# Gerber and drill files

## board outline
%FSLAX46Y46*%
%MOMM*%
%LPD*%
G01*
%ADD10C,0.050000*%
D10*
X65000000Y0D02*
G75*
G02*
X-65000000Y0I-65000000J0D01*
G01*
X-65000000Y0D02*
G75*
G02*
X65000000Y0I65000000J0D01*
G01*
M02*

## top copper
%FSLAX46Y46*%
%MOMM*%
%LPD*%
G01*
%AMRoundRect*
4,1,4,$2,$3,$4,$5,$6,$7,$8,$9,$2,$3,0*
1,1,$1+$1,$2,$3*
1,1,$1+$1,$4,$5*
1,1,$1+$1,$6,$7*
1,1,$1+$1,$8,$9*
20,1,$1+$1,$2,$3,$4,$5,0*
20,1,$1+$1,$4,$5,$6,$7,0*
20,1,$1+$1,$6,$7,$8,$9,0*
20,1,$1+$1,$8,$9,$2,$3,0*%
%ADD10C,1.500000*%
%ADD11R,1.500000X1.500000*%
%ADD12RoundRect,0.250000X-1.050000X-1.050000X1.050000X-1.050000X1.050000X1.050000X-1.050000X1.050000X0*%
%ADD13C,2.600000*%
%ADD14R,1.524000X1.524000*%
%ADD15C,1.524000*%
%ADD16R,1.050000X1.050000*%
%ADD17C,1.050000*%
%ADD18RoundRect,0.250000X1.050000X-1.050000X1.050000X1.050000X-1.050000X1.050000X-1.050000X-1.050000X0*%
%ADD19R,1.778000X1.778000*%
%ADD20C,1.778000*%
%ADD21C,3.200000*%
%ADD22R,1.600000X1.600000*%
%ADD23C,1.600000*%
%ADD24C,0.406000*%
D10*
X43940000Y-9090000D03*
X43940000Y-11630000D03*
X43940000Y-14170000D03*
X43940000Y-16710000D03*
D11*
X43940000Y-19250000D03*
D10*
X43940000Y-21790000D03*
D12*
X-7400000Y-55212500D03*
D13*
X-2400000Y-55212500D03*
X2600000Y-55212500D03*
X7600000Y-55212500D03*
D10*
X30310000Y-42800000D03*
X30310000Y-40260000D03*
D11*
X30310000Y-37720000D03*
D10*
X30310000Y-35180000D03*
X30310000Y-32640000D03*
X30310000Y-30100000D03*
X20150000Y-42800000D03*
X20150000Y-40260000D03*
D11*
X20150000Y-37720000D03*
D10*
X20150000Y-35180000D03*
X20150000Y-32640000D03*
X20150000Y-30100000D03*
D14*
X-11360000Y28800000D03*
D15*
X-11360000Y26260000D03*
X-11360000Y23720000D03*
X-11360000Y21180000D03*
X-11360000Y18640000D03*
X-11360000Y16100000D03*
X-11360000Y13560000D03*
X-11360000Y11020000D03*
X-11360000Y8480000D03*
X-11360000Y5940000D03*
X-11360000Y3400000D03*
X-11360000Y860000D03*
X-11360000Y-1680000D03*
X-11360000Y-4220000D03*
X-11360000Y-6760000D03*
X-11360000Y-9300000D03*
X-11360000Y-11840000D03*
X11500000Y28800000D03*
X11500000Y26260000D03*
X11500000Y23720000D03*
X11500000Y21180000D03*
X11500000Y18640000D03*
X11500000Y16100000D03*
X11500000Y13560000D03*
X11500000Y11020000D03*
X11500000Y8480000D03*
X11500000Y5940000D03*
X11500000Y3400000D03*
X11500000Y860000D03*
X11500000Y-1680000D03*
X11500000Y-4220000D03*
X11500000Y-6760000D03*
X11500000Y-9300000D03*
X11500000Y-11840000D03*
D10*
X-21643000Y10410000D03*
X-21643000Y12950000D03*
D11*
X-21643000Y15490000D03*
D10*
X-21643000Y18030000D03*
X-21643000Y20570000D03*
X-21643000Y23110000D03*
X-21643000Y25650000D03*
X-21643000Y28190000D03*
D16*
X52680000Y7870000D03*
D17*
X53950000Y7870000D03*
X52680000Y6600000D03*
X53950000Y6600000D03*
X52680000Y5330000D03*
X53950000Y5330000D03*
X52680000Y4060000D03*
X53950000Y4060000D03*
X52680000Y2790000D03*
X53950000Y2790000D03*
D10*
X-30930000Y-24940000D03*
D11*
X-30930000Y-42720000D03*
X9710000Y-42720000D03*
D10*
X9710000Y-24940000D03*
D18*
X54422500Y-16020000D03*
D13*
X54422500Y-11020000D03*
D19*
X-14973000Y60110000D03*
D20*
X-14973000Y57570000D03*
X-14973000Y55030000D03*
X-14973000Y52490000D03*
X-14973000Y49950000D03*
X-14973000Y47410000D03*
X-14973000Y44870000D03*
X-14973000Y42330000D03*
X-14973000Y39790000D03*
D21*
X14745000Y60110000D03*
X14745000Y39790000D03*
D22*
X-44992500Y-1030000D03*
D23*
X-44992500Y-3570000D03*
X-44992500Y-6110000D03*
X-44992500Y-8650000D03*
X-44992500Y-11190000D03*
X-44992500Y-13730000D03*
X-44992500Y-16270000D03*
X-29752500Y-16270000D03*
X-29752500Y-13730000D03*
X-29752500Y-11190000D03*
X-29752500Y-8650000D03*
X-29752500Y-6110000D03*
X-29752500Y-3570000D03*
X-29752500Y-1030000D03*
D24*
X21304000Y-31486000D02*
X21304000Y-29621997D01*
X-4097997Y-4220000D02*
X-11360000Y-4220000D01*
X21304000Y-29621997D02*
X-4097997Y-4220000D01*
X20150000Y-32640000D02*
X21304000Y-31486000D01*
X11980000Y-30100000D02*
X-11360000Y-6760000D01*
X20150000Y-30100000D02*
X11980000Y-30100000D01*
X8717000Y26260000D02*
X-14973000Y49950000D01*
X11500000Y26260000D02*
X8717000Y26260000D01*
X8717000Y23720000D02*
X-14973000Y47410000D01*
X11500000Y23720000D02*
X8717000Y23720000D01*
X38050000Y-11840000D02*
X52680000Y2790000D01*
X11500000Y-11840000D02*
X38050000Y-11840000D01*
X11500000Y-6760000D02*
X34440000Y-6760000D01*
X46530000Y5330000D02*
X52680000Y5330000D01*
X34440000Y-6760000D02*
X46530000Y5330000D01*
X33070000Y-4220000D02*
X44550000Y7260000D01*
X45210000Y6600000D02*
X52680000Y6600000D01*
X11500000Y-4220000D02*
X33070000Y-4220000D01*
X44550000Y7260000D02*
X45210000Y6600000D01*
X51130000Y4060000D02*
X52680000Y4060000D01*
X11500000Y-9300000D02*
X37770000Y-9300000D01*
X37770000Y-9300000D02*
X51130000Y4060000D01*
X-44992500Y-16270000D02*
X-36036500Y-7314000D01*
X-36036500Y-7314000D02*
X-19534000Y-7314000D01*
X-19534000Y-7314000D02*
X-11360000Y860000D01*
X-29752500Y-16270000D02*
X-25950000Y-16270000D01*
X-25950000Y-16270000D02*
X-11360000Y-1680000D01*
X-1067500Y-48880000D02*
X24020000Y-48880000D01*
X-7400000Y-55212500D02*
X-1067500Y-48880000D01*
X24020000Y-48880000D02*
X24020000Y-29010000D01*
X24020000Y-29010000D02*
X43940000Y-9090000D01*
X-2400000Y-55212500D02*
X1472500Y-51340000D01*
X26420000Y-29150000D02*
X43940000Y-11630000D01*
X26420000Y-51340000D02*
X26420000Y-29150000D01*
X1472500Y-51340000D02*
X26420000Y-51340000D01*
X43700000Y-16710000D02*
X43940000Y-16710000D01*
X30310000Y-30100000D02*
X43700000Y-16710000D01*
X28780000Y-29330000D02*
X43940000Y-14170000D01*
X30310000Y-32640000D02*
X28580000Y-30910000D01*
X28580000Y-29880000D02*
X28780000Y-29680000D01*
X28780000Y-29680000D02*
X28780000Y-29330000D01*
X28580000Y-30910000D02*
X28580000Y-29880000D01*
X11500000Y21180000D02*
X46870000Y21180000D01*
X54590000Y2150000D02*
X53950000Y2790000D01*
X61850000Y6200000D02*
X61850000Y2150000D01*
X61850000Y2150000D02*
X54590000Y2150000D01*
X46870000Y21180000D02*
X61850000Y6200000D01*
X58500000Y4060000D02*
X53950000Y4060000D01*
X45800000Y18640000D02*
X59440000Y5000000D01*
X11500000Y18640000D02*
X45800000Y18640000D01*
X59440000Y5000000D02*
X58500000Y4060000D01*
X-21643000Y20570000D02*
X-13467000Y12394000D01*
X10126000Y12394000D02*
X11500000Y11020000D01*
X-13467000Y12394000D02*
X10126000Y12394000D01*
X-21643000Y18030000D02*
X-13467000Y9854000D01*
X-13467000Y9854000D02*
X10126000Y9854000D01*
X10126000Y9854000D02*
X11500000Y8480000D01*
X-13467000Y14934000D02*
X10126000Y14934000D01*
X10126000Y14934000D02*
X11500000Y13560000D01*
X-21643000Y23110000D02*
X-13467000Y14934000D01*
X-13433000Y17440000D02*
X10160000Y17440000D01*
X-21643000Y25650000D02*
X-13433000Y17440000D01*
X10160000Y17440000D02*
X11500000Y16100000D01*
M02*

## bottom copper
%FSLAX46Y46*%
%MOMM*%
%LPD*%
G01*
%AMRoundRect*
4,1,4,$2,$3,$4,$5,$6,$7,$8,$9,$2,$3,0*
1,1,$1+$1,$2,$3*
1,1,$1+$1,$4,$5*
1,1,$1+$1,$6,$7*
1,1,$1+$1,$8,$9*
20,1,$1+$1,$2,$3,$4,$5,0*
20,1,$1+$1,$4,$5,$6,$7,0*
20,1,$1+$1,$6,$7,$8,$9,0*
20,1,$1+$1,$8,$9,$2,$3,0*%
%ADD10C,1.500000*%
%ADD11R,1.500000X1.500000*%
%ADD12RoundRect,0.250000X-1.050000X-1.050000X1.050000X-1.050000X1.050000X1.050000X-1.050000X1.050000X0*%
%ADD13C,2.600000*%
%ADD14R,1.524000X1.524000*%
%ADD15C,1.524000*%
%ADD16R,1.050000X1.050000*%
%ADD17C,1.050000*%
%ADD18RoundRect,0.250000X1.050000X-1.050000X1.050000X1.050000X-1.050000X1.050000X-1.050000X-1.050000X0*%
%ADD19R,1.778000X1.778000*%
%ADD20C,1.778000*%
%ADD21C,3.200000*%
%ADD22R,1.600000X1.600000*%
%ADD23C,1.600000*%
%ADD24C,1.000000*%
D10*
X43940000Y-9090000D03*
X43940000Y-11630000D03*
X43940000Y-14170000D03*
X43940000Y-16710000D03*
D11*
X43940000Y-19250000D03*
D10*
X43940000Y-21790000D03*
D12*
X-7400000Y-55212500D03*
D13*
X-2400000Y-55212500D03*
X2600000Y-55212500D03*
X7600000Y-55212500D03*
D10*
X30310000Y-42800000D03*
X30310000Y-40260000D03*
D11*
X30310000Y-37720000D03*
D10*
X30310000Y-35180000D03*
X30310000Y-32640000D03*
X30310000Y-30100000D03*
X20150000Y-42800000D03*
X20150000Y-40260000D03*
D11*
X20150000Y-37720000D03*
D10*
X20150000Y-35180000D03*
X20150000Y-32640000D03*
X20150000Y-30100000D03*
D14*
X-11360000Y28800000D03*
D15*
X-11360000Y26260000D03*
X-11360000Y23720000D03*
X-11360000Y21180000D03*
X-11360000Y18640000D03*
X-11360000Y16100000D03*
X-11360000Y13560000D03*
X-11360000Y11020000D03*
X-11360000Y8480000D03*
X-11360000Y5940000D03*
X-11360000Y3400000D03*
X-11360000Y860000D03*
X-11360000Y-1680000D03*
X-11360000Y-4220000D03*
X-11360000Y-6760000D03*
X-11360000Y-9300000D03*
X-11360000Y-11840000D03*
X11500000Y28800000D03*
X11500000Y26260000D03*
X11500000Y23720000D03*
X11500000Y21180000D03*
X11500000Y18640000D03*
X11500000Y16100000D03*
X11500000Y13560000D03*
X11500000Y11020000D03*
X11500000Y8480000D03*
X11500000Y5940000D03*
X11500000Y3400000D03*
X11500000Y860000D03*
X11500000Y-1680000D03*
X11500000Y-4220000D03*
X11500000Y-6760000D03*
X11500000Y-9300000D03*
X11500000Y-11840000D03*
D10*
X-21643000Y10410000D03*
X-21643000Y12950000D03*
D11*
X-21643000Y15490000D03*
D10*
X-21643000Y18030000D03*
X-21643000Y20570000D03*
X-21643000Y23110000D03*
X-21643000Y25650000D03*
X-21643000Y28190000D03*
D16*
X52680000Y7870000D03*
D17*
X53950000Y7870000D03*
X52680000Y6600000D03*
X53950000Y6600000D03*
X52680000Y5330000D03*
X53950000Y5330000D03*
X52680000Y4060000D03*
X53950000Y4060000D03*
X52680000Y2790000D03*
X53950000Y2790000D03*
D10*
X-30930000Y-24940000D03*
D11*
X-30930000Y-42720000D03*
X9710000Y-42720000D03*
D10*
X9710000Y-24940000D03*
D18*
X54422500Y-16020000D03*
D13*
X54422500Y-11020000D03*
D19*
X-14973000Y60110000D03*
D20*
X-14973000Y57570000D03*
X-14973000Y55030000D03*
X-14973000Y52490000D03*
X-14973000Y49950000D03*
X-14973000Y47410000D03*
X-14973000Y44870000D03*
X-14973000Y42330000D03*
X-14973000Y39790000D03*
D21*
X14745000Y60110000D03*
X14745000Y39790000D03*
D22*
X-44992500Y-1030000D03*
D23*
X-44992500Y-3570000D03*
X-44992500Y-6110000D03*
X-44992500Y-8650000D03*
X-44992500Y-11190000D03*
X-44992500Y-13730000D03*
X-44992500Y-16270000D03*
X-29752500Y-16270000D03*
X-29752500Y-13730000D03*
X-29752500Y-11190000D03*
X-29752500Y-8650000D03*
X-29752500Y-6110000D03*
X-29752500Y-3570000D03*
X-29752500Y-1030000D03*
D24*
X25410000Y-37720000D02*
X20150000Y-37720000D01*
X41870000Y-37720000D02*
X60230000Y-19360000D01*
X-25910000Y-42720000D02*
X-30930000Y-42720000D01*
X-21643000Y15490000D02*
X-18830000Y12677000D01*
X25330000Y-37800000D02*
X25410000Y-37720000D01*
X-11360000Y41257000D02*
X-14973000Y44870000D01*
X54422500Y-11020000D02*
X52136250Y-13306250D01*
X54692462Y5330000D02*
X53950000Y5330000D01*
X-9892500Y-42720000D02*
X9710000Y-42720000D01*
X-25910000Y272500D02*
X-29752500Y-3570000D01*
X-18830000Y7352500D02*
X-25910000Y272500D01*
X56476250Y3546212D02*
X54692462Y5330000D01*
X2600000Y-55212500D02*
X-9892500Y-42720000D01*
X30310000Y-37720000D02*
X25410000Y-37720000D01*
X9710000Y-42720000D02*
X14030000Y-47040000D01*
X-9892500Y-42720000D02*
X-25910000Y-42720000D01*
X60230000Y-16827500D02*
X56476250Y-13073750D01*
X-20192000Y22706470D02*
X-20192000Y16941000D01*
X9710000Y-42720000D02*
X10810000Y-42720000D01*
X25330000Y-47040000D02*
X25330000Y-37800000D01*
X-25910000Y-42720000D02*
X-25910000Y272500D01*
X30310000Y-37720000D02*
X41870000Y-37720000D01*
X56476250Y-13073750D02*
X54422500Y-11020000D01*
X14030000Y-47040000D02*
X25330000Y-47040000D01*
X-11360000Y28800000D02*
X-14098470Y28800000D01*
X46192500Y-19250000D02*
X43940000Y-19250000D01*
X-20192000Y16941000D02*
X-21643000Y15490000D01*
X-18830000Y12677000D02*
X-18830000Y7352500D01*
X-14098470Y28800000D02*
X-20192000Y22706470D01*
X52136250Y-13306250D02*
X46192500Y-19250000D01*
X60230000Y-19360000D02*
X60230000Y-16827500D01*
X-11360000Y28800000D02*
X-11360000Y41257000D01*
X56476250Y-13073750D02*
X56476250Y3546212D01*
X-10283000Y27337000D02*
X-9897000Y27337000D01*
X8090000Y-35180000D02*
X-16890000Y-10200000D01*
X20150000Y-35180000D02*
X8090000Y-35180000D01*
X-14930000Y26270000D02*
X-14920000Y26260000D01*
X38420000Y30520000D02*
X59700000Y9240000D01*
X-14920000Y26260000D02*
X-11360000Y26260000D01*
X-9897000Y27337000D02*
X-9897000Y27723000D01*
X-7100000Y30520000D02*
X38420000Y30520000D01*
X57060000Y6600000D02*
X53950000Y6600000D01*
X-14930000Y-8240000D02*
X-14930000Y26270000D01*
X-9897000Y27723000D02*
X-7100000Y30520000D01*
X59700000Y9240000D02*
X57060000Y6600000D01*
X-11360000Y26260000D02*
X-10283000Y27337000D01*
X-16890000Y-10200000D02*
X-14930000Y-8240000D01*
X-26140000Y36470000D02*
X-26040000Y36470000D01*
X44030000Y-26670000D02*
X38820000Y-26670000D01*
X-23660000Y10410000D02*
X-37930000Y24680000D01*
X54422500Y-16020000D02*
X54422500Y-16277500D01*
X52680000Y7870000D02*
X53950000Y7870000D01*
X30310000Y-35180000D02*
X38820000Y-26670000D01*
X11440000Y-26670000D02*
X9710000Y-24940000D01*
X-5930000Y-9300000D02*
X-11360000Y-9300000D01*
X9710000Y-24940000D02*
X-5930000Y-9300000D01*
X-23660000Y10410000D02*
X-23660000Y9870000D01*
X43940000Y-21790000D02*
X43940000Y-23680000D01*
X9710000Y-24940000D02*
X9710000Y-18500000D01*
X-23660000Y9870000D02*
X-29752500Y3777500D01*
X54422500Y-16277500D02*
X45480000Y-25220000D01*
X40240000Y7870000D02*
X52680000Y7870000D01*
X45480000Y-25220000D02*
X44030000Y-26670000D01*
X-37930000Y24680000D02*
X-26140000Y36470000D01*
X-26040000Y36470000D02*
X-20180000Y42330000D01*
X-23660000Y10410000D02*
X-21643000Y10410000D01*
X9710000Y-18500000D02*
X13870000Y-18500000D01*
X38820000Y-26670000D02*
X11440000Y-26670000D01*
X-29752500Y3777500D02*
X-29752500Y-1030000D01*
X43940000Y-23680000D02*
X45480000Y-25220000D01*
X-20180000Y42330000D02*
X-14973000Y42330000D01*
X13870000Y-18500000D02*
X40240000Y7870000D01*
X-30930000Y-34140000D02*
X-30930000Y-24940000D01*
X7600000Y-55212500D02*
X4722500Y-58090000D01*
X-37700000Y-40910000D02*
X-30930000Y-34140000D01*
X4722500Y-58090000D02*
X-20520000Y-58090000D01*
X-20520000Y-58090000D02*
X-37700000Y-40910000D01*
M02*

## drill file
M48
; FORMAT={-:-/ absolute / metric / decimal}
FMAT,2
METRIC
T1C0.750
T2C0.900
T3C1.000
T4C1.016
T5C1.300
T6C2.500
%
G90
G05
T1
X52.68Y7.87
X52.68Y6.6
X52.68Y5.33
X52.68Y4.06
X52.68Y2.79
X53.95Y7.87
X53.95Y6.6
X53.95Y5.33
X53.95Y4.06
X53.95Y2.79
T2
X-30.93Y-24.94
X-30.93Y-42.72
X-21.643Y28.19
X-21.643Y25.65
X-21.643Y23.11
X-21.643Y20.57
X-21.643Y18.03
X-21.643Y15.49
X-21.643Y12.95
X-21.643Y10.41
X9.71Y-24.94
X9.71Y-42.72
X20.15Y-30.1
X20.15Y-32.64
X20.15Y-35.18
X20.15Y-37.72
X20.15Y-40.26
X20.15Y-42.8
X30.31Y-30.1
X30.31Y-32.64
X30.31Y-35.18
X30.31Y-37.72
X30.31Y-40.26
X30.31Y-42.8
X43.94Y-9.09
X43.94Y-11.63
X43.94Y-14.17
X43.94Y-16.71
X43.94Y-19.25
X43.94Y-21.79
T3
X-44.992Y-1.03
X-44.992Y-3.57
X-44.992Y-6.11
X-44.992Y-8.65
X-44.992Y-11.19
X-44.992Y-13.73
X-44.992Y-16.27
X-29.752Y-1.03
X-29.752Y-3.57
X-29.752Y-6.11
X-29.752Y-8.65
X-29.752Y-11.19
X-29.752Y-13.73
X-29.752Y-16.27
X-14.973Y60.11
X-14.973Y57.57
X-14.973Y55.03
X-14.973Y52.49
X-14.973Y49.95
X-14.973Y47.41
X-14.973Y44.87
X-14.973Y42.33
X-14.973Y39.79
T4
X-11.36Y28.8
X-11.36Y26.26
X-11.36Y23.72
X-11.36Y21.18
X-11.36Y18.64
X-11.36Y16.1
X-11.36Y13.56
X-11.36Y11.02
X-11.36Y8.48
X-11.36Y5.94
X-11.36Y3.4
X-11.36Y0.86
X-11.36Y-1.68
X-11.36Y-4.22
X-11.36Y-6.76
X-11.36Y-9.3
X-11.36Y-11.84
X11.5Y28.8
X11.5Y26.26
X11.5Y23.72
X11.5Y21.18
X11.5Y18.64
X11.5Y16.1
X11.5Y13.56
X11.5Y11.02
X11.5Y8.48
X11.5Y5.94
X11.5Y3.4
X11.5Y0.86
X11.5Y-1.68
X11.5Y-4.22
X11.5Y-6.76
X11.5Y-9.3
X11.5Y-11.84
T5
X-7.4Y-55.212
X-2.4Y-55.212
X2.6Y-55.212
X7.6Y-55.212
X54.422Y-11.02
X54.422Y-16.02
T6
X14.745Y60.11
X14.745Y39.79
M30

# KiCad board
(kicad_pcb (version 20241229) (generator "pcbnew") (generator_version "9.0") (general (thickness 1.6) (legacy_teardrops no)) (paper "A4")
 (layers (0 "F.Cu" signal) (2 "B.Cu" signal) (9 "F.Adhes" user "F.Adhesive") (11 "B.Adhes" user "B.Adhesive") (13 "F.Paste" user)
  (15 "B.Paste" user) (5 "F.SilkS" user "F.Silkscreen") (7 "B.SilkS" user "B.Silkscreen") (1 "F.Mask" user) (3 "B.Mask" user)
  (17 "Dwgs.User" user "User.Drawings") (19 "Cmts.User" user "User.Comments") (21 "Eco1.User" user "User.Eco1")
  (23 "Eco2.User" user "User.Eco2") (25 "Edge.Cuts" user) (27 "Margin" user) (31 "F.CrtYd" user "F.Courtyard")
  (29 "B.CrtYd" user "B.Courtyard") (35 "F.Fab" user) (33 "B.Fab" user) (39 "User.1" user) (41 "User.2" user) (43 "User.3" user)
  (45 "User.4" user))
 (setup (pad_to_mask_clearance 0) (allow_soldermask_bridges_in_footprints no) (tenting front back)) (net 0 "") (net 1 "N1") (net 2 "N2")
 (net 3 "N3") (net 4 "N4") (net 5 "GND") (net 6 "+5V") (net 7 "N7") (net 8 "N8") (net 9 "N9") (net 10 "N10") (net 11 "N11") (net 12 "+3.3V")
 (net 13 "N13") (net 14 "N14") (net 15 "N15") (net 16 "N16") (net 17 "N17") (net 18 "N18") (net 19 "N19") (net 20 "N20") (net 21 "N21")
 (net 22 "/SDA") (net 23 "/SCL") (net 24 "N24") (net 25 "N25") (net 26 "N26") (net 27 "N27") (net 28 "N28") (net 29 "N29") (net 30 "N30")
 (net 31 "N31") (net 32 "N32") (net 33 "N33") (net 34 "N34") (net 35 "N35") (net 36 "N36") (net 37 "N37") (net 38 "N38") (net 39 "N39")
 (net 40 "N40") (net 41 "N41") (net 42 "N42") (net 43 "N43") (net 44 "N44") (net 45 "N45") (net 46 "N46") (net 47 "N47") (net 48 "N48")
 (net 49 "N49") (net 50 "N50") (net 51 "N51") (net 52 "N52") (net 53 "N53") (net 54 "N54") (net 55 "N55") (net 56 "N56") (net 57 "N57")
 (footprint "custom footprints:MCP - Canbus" (layer "F.Cu") (at 43.94 21.79)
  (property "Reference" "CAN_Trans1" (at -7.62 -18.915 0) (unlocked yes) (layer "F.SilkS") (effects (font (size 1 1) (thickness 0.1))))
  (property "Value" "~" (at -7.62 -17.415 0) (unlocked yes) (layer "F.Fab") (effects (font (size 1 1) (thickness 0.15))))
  (pad "1" thru_hole circle (at 0 -12.7 180) (size 1.5 1.5) (drill 0.9) (layers "*.Cu" "*.Mask") (remove_unused_layers no) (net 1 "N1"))
  (pad "2" thru_hole circle (at 0 -10.16 180) (size 1.5 1.5) (drill 0.9) (layers "*.Cu" "*.Mask") (remove_unused_layers no) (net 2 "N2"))
  (pad "3" thru_hole circle (at 0 -7.62 180) (size 1.5 1.5) (drill 0.9) (layers "*.Cu" "*.Mask") (remove_unused_layers no) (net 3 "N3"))
  (pad "4" thru_hole circle (at 0 -5.08 180) (size 1.5 1.5) (drill 0.9) (layers "*.Cu" "*.Mask") (remove_unused_layers no) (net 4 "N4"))
  (pad "5" thru_hole rect (at 0 -2.54 180) (size 1.5 1.5) (drill 0.9) (layers "*.Cu" "*.Mask") (remove_unused_layers no) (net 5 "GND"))
  (pad "6" thru_hole circle (at 0 0 180) (size 1.5 1.5) (drill 0.9) (layers "*.Cu" "*.Mask") (remove_unused_layers no) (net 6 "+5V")))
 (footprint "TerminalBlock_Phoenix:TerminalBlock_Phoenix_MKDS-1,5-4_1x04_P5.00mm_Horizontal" (layer "F.Cu") (at -7.4 55.2125)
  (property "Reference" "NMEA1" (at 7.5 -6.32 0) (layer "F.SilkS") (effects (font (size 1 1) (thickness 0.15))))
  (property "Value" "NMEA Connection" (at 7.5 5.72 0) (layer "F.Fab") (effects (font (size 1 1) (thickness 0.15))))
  (pad "1" thru_hole roundrect (at 0 0) (size 2.6 2.6) (drill 1.3) (layers "*.Cu" "*.Mask") (remove_unused_layers no)
   (roundrect_rratio 0.096154) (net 1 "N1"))
  (pad "2" thru_hole circle (at 5 0) (size 2.6 2.6) (drill 1.3) (layers "*.Cu" "*.Mask") (remove_unused_layers no) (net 2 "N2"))
  (pad "3" thru_hole circle (at 10 0) (size 2.6 2.6) (drill 1.3) (layers "*.Cu" "*.Mask") (remove_unused_layers no) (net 5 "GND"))
  (pad "4" thru_hole circle (at 15 0) (size 2.6 2.6) (drill 1.3) (layers "*.Cu" "*.Mask") (remove_unused_layers no) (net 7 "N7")))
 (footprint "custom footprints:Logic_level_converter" (layer "F.Cu") (at 30.31 30.1 180)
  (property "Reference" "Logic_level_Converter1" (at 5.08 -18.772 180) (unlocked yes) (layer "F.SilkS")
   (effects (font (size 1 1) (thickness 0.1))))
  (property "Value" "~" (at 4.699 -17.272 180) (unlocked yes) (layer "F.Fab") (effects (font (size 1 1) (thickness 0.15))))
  (pad "1" thru_hole circle (at 0 -12.7) (size 1.5 1.5) (drill 0.9) (layers "*.Cu" "*.Mask") (remove_unused_layers no) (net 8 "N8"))
  (pad "2" thru_hole circle (at 0 -10.16) (size 1.5 1.5) (drill 0.9) (layers "*.Cu" "*.Mask") (remove_unused_layers no) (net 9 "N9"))
  (pad "3" thru_hole rect (at 0 -7.62) (size 1.5 1.5) (drill 0.9) (layers "*.Cu" "*.Mask") (remove_unused_layers no) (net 5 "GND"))
  (pad "4" thru_hole circle (at 0 -5.08) (size 1.5 1.5) (drill 0.9) (layers "*.Cu" "*.Mask") (remove_unused_layers no) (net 6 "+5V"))
  (pad "5" thru_hole circle (at 0 -2.54) (size 1.5 1.5) (drill 0.9) (layers "*.Cu" "*.Mask") (remove_unused_layers no) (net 3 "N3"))
  (pad "6" thru_hole circle (at 0 0) (size 1.5 1.5) (drill 0.9) (layers "*.Cu" "*.Mask") (remove_unused_layers no) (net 4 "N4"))
  (pad "7" thru_hole circle (at 10.16 -12.7) (size 1.5 1.5) (drill 0.9) (layers "*.Cu" "*.Mask") (remove_unused_layers no) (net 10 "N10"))
  (pad "8" thru_hole circle (at 10.16 -10.16) (size 1.5 1.5) (drill 0.9) (layers "*.Cu" "*.Mask") (remove_unused_layers no) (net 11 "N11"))
  (pad "9" thru_hole rect (at 10.16 -7.62) (size 1.5 1.5) (drill 0.9) (layers "*.Cu" "*.Mask") (remove_unused_layers no) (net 5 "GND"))
  (pad "10" thru_hole circle (at 10.16 -5.08) (size 1.5 1.5) (drill 0.9) (layers "*.Cu" "*.Mask") (remove_unused_layers no) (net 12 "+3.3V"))
  (pad "11" thru_hole circle (at 10.16 -2.54) (size 1.5 1.5) (drill 0.9) (layers "*.Cu" "*.Mask") (remove_unused_layers no) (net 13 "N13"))
  (pad "12" thru_hole circle (at 10.16 0) (size 1.5 1.5) (drill 0.9) (layers "*.Cu" "*.Mask") (remove_unused_layers no) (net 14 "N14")))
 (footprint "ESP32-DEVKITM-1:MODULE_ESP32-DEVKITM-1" (layer "F.Cu") (at 0.07 -8.465)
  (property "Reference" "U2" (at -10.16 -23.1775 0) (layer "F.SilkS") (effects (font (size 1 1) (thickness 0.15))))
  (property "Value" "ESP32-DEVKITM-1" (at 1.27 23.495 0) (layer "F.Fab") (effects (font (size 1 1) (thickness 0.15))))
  (pad "J1_1" thru_hole rect (at -11.43 -20.335) (size 1.524 1.524) (drill 1.016) (layers "*.Cu" "*.Mask") (remove_unused_layers no)
   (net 5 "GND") (solder_mask_margin 0.102))
  (pad "J1_2" thru_hole circle (at -11.43 -17.795) (size 1.524 1.524) (drill 1.016) (layers "*.Cu" "*.Mask") (remove_unused_layers no)
   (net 12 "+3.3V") (solder_mask_margin 0.102))
  (pad "J1_3" thru_hole circle (at -11.43 -15.255) (size 1.524 1.524) (drill 1.016) (layers "*.Cu" "*.Mask") (remove_unused_layers no)
   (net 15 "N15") (solder_mask_margin 0.102))
  (pad "J1_4" thru_hole circle (at -11.43 -12.715) (size 1.524 1.524) (drill 1.016) (layers "*.Cu" "*.Mask") (remove_unused_layers no)
   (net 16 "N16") (solder_mask_margin 0.102))
  (pad "J1_5" thru_hole circle (at -11.43 -10.175) (size 1.524 1.524) (drill 1.016) (layers "*.Cu" "*.Mask") (remove_unused_layers no)
   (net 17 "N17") (solder_mask_margin 0.102))
  (pad "J1_6" thru_hole circle (at -11.43 -7.635) (size 1.524 1.524) (drill 1.016) (layers "*.Cu" "*.Mask") (remove_unused_layers no)
   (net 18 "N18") (solder_mask_margin 0.102))
  (pad "J1_7" thru_hole circle (at -11.43 -5.095) (size 1.524 1.524) (drill 1.016) (layers "*.Cu" "*.Mask") (remove_unused_layers no)
   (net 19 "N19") (solder_mask_margin 0.102))
  (pad "J1_8" thru_hole circle (at -11.43 -2.555) (size 1.524 1.524) (drill 1.016) (layers "*.Cu" "*.Mask") (remove_unused_layers no)
   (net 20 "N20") (solder_mask_margin 0.102))
  (pad "J1_9" thru_hole circle (at -11.43 -0.015) (size 1.524 1.524) (drill 1.016) (layers "*.Cu" "*.Mask") (remove_unused_layers no)
   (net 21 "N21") (solder_mask_margin 0.102))
  (pad "J1_10" thru_hole circle (at -11.43 2.525) (size 1.524 1.524) (drill 1.016) (layers "*.Cu" "*.Mask") (remove_unused_layers no)
   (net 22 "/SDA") (solder_mask_margin 0.102))
  (pad "J1_11" thru_hole circle (at -11.43 5.065) (size 1.524 1.524) (drill 1.016) (layers "*.Cu" "*.Mask") (remove_unused_layers no)
   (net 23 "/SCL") (solder_mask_margin 0.102))
  (pad "J1_12" thru_hole circle (at -11.43 7.605) (size 1.524 1.524) (drill 1.016) (layers "*.Cu" "*.Mask") (remove_unused_layers no)
   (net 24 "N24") (solder_mask_margin 0.102))
  (pad "J1_13" thru_hole circle (at -11.43 10.145) (size 1.524 1.524) (drill 1.016) (layers "*.Cu" "*.Mask") (remove_unused_layers no)
   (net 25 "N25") (solder_mask_margin 0.102))
  (pad "J1_14" thru_hole circle (at -11.43 12.685) (size 1.524 1.524) (drill 1.016) (layers "*.Cu" "*.Mask") (remove_unused_layers no)
   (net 13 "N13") (solder_mask_margin 0.102))
  (pad "J1_15" thru_hole circle (at -11.43 15.225) (size 1.524 1.524) (drill 1.016) (layers "*.Cu" "*.Mask") (remove_unused_layers no)
   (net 14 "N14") (solder_mask_margin 0.102))
  (pad "J1_16" thru_hole circle (at -11.43 17.765) (size 1.524 1.524) (drill 1.016) (layers "*.Cu" "*.Mask") (remove_unused_layers no)
   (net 6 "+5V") (solder_mask_margin 0.102))
  (pad "J1_17" thru_hole circle (at -11.43 20.305) (size 1.524 1.524) (drill 1.016) (layers "*.Cu" "*.Mask") (remove_unused_layers no)
   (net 5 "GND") (solder_mask_margin 0.102))
  (pad "J3_1" thru_hole circle (at 11.43 -20.335) (size 1.524 1.524) (drill 1.016) (layers "*.Cu" "*.Mask") (remove_unused_layers no)
   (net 5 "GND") (solder_mask_margin 0.102))
  (pad "J3_2" thru_hole circle (at 11.43 -17.795) (size 1.524 1.524) (drill 1.016) (layers "*.Cu" "*.Mask") (remove_unused_layers no)
   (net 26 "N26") (solder_mask_margin 0.102))
  (pad "J3_3" thru_hole circle (at 11.43 -15.255) (size 1.524 1.524) (drill 1.016) (layers "*.Cu" "*.Mask") (remove_unused_layers no)
   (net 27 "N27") (solder_mask_margin 0.102))
  (pad "J3_4" thru_hole circle (at 11.43 -12.715) (size 1.524 1.524) (drill 1.016) (layers "*.Cu" "*.Mask") (remove_unused_layers no)
   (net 22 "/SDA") (solder_mask_margin 0.102))
  (pad "J3_5" thru_hole circle (at 11.43 -10.175) (size 1.524 1.524) (drill 1.016) (layers "*.Cu" "*.Mask") (remove_unused_layers no)
   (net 23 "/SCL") (solder_mask_margin 0.102))
  (pad "J3_6" thru_hole circle (at 11.43 -7.635) (size 1.524 1.524) (drill 1.016) (layers "*.Cu" "*.Mask") (remove_unused_layers no)
   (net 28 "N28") (solder_mask_margin 0.102))
  (pad "J3_7" thru_hole circle (at 11.43 -5.095) (size 1.524 1.524) (drill 1.016) (layers "*.Cu" "*.Mask") (remove_unused_layers no)
   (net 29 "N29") (solder_mask_margin 0.102))
  (pad "J3_8" thru_hole circle (at 11.43 -2.555) (size 1.524 1.524) (drill 1.016) (layers "*.Cu" "*.Mask") (remove_unused_layers no)
   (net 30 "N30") (solder_mask_margin 0.102))
  (pad "J3_9" thru_hole circle (at 11.43 -0.015) (size 1.524 1.524) (drill 1.016) (layers "*.Cu" "*.Mask") (remove_unused_layers no)
   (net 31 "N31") (solder_mask_margin 0.102))
  (pad "J3_10" thru_hole circle (at 11.43 2.525) (size 1.524 1.524) (drill 1.016) (layers "*.Cu" "*.Mask") (remove_unused_layers no)
   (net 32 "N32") (solder_mask_margin 0.102))
  (pad "J3_11" thru_hole circle (at 11.43 5.065) (size 1.524 1.524) (drill 1.016) (layers "*.Cu" "*.Mask") (remove_unused_layers no)
   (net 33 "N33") (solder_mask_margin 0.102))
  (pad "J3_12" thru_hole circle (at 11.43 7.605) (size 1.524 1.524) (drill 1.016) (layers "*.Cu" "*.Mask") (remove_unused_layers no)
   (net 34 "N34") (solder_mask_margin 0.102))
  (pad "J3_13" thru_hole circle (at 11.43 10.145) (size 1.524 1.524) (drill 1.016) (layers "*.Cu" "*.Mask") (remove_unused_layers no)
   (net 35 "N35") (solder_mask_margin 0.102))
  (pad "J3_14" thru_hole circle (at 11.43 12.685) (size 1.524 1.524) (drill 1.016) (layers "*.Cu" "*.Mask") (remove_unused_layers no)
   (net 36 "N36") (solder_mask_margin 0.102))
  (pad "J3_15" thru_hole circle (at 11.43 15.225) (size 1.524 1.524) (drill 1.016) (layers "*.Cu" "*.Mask") (remove_unused_layers no)
   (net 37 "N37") (solder_mask_margin 0.102))
  (pad "J3_16" thru_hole circle (at 11.43 17.765) (size 1.524 1.524) (drill 1.016) (layers "*.Cu" "*.Mask") (remove_unused_layers no)
   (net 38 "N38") (solder_mask_margin 0.102))
  (pad "J3_17" thru_hole circle (at 11.43 20.305) (size 1.524 1.524) (drill 1.016) (layers "*.Cu" "*.Mask") (remove_unused_layers no)
   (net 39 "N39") (solder_mask_margin 0.102)))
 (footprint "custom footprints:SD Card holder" (layer "F.Cu") (at -21.643 -10.41)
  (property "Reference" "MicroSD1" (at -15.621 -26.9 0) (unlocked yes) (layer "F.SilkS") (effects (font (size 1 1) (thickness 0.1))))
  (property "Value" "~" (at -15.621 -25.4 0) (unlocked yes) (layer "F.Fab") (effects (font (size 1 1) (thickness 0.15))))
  (pad "1" thru_hole circle (at 0 0 180) (size 1.5 1.5) (drill 0.9) (layers "*.Cu" "*.Mask") (remove_unused_layers no) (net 6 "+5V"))
  (pad "2" thru_hole circle (at 0 -2.54 180) (size 1.5 1.5) (drill 0.9) (layers "*.Cu" "*.Mask") (remove_unused_layers no) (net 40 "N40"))
  (pad "3" thru_hole rect (at 0 -5.08 180) (size 1.5 1.5) (drill 0.9) (layers "*.Cu" "*.Mask") (remove_unused_layers no) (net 5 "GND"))
  (pad "4" thru_hole circle (at 0 -7.62 180) (size 1.5 1.5) (drill 0.9) (layers "*.Cu" "*.Mask") (remove_unused_layers no) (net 31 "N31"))
  (pad "5" thru_hole circle (at 0 -10.16 180) (size 1.5 1.5) (drill 0.9) (layers "*.Cu" "*.Mask") (remove_unused_layers no) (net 30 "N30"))
  (pad "6" thru_hole circle (at 0 -12.7 180) (size 1.5 1.5) (drill 0.9) (layers "*.Cu" "*.Mask") (remove_unused_layers no) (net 29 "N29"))
  (pad "7" thru_hole circle (at 0 -15.24 180) (size 1.5 1.5) (drill 0.9) (layers "*.Cu" "*.Mask") (remove_unused_layers no) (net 28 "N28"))
  (pad "8" thru_hole circle (at 0 -17.78 180) (size 1.5 1.5) (drill 0.9) (layers "*.Cu" "*.Mask") (remove_unused_layers no) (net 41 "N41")))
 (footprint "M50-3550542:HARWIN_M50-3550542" (layer "F.Cu") (at 53.315 -5.33 -90)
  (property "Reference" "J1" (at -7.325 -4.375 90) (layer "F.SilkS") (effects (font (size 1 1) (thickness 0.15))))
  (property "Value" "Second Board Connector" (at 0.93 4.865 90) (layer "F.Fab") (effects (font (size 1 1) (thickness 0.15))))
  (pad "1" thru_hole rect (at -2.54 0.635 270) (size 1.05 1.05) (drill 0.75) (layers "*.Cu" "*.Mask") (remove_unused_layers no)
   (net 6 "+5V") (solder_mask_margin 0.102))
  (pad "2" thru_hole circle (at -2.54 -0.635 270) (size 1.05 1.05) (drill 0.75) (layers "*.Cu" "*.Mask") (remove_unused_layers no)
   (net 6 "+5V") (solder_mask_margin 0.102))
  (pad "3" thru_hole circle (at -1.27 0.635 270) (size 1.05 1.05) (drill 0.75) (layers "*.Cu" "*.Mask") (remove_unused_layers no)
   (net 36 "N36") (solder_mask_margin 0.102))
  (pad "4" thru_hole circle (at -1.27 -0.635 270) (size 1.05 1.05) (drill 0.75) (layers "*.Cu" "*.Mask") (remove_unused_layers no)
   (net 12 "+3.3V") (solder_mask_margin 0.102))
  (pad "5" thru_hole circle (at 0 0.635 270) (size 1.05 1.05) (drill 0.75) (layers "*.Cu" "*.Mask") (remove_unused_layers no) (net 37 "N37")
   (solder_mask_margin 0.102))
  (pad "6" thru_hole circle (at 0 -0.635 270) (size 1.05 1.05) (drill 0.75) (layers "*.Cu" "*.Mask") (remove_unused_layers no) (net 5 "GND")
   (solder_mask_margin 0.102))
  (pad "7" thru_hole circle (at 1.27 0.635 270) (size 1.05 1.05) (drill 0.75) (layers "*.Cu" "*.Mask") (remove_unused_layers no)
   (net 38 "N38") (solder_mask_margin 0.102))
  (pad "8" thru_hole circle (at 1.27 -0.635 270) (size 1.05 1.05) (drill 0.75) (layers "*.Cu" "*.Mask") (remove_unused_layers no)
   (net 23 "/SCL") (solder_mask_margin 0.102))
  (pad "9" thru_hole circle (at 2.54 0.635 270) (size 1.05 1.05) (drill 0.75) (layers "*.Cu" "*.Mask") (remove_unused_layers no)
   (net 39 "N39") (solder_mask_margin 0.102))
  (pad "10" thru_hole circle (at 2.54 -0.635 270) (size 1.05 1.05) (drill 0.75) (layers "*.Cu" "*.Mask") (remove_unused_layers no)
   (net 22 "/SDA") (solder_mask_margin 0.102)))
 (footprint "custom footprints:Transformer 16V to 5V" (layer "F.Cu") (at -30.93 42.72)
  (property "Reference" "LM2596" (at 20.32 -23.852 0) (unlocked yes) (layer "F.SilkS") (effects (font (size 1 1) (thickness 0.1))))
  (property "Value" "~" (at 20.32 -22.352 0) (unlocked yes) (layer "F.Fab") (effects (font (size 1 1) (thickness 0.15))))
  (pad "1" thru_hole circle (at 0 -17.78) (size 1.5 1.5) (drill 0.9) (layers "*.Cu" "*.Mask") (remove_unused_layers no) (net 7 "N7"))
  (pad "2" thru_hole rect (at 0 0) (size 1.5 1.5) (drill 0.9) (layers "*.Cu" "*.Mask") (remove_unused_layers no) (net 5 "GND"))
  (pad "3" thru_hole rect (at 40.64 0) (size 1.5 1.5) (drill 0.9) (layers "*.Cu" "*.Mask") (remove_unused_layers no) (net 5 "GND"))
  (pad "4" thru_hole circle (at 40.64 -17.78) (size 1.5 1.5) (drill 0.9) (layers "*.Cu" "*.Mask") (remove_unused_layers no) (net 6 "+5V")))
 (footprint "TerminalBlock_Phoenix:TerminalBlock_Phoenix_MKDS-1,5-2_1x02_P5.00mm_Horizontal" (layer "F.Cu") (at 54.4225 16.02 90)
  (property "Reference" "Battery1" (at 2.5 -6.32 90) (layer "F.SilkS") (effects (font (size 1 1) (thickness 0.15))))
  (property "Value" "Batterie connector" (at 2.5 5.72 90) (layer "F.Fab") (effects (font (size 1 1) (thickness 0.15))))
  (pad "1" thru_hole roundrect (at 0 0 90) (size 2.6 2.6) (drill 1.3) (layers "*.Cu" "*.Mask") (remove_unused_layers no)
   (roundrect_rratio 0.096154) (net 6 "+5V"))
  (pad "2" thru_hole circle (at 5 0 90) (size 2.6 2.6) (drill 1.3) (layers "*.Cu" "*.Mask") (remove_unused_layers no) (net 5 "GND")))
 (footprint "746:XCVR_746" (layer "F.Cu") (at 0.14 -49.95 -90)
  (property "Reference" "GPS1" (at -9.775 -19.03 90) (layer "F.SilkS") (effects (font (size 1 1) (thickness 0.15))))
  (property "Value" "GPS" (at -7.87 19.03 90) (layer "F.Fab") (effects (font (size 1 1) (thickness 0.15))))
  (pad "1" thru_hole rect (at -10.16 15.113 270) (size 1.778 1.778) (drill 1) (layers "*.Cu" "*.Mask") (remove_unused_layers no)
   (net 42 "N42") (solder_mask_margin 0.102))
  (pad "2" thru_hole circle (at -7.62 15.113 270) (size 1.778 1.778) (drill 1) (layers "*.Cu" "*.Mask") (remove_unused_layers no)
   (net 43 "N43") (solder_mask_margin 0.102))
  (pad "3" thru_hole circle (at -5.08 15.113 270) (size 1.778 1.778) (drill 1) (layers "*.Cu" "*.Mask") (remove_unused_layers no)
   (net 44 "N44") (solder_mask_margin 0.102))
  (pad "4" thru_hole circle (at -2.54 15.113 270) (size 1.778 1.778) (drill 1) (layers "*.Cu" "*.Mask") (remove_unused_layers no)
   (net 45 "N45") (solder_mask_margin 0.102))
  (pad "5" thru_hole circle (at 0 15.113 270) (size 1.778 1.778) (drill 1) (layers "*.Cu" "*.Mask") (remove_unused_layers no) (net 26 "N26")
   (solder_mask_margin 0.102))
  (pad "6" thru_hole circle (at 2.54 15.113 270) (size 1.778 1.778) (drill 1) (layers "*.Cu" "*.Mask") (remove_unused_layers no)
   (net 27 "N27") (solder_mask_margin 0.102))
  (pad "7" thru_hole circle (at 5.08 15.113 270) (size 1.778 1.778) (drill 1) (layers "*.Cu" "*.Mask") (remove_unused_layers no)
   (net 5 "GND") (solder_mask_margin 0.102))
  (pad "8" thru_hole circle (at 7.62 15.113 270) (size 1.778 1.778) (drill 1) (layers "*.Cu" "*.Mask") (remove_unused_layers no)
   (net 6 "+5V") (solder_mask_margin 0.102))
  (pad "9" thru_hole circle (at 10.16 15.113 270) (size 1.778 1.778) (drill 1) (layers "*.Cu" "*.Mask") (remove_unused_layers no)
   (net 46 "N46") (solder_mask_margin 0.102))
  (pad "SH1" thru_hole circle (at -10.16 -14.605 270) (size 3.2 3.2) (drill 2.5) (layers "*.Cu" "*.Mask") (remove_unused_layers no)
   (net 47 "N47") (solder_mask_margin 0.102))
  (pad "SH2" thru_hole circle (at 10.16 -14.605 270) (size 3.2 3.2) (drill 2.5) (layers "*.Cu" "*.Mask") (remove_unused_layers no)
   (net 47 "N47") (solder_mask_margin 0.102)))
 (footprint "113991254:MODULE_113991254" (layer "F.Cu") (at -37.3725 8.65)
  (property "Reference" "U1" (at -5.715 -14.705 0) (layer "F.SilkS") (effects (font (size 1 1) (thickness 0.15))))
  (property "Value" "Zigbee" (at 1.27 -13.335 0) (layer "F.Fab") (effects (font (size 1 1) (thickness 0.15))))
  (pad "1" thru_hole rect (at -7.62 -7.62) (size 1.6 1.6) (drill 1) (layers "*.Cu" "*.Mask") (remove_unused_layers no) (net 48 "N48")
   (solder_mask_margin 0.102))
  (pad "2" thru_hole circle (at -7.62 -5.08) (size 1.6 1.6) (drill 1) (layers "*.Cu" "*.Mask") (remove_unused_layers no) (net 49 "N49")
   (solder_mask_margin 0.102))
  (pad "3" thru_hole circle (at -7.62 -2.54) (size 1.6 1.6) (drill 1) (layers "*.Cu" "*.Mask") (remove_unused_layers no) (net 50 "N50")
   (solder_mask_margin 0.102))
  (pad "4" thru_hole circle (at -7.62 0) (size 1.6 1.6) (drill 1) (layers "*.Cu" "*.Mask") (remove_unused_layers no) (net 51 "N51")
   (solder_mask_margin 0.102))
  (pad "5" thru_hole circle (at -7.62 2.54) (size 1.6 1.6) (drill 1) (layers "*.Cu" "*.Mask") (remove_unused_layers no) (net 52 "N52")
   (solder_mask_margin 0.102))
  (pad "6" thru_hole circle (at -7.62 5.08) (size 1.6 1.6) (drill 1) (layers "*.Cu" "*.Mask") (remove_unused_layers no) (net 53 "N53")
   (solder_mask_margin 0.102))
  (pad "7" thru_hole circle (at -7.62 7.62) (size 1.6 1.6) (drill 1) (layers "*.Cu" "*.Mask") (remove_unused_layers no) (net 24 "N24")
   (solder_mask_margin 0.102))
  (pad "8" thru_hole circle (at 7.62 7.62) (size 1.6 1.6) (drill 1) (layers "*.Cu" "*.Mask") (remove_unused_layers no) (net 25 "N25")
   (solder_mask_margin 0.102))
  (pad "9" thru_hole circle (at 7.62 5.08) (size 1.6 1.6) (drill 1) (layers "*.Cu" "*.Mask") (remove_unused_layers no) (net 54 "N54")
   (solder_mask_margin 0.102))
  (pad "10" thru_hole circle (at 7.62 2.54) (size 1.6 1.6) (drill 1) (layers "*.Cu" "*.Mask") (remove_unused_layers no) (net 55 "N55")
   (solder_mask_margin 0.102))
  (pad "11" thru_hole circle (at 7.62 0) (size 1.6 1.6) (drill 1) (layers "*.Cu" "*.Mask") (remove_unused_layers no) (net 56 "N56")
   (solder_mask_margin 0.102))
  (pad "12" thru_hole circle (at 7.62 -2.54) (size 1.6 1.6) (drill 1) (layers "*.Cu" "*.Mask") (remove_unused_layers no) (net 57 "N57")
   (solder_mask_margin 0.102))
  (pad "13" thru_hole circle (at 7.62 -5.08) (size 1.6 1.6) (drill 1) (layers "*.Cu" "*.Mask") (remove_unused_layers no) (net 5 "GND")
   (solder_mask_margin 0.102))
  (pad "14" thru_hole circle (at 7.62 -7.62) (size 1.6 1.6) (drill 1) (layers "*.Cu" "*.Mask") (remove_unused_layers no) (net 6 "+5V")
   (solder_mask_margin 0.102)))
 (gr_circle (center 0 0) (end 65 0) (stroke (width 0.05) (type solid)) (fill no) (layer "Edge.Cuts"))
 (segment (start 25.41 37.72) (end 20.15 37.72) (width 1) (layer "B.Cu") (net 5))
 (segment (start 41.87 37.72) (end 60.23 19.36) (width 1) (layer "B.Cu") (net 5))
 (segment (start -25.91 42.72) (end -30.93 42.72) (width 1) (layer "B.Cu") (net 5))
 (segment (start -21.643 -15.49) (end -18.83 -12.677) (width 1) (layer "B.Cu") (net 5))
 (segment (start 25.33 37.8) (end 25.41 37.72) (width 1) (layer "B.Cu") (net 5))
 (segment (start -11.36 -41.257) (end -14.973 -44.87) (width 1) (layer "B.Cu") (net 5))
 (segment (start 54.4225 11.02) (end 52.13625 13.30625) (width 1) (layer "B.Cu") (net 5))
 (segment (start 54.692462 -5.33) (end 53.95 -5.33) (width 1) (layer "B.Cu") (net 5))
 (segment (start -9.8925 42.72) (end 9.71 42.72) (width 1) (layer "B.Cu") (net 5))
 (segment (start -25.91 -0.2725) (end -29.7525 3.57) (width 1) (layer "B.Cu") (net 5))
 (segment (start -18.83 -7.3525) (end -25.91 -0.2725) (width 1) (layer "B.Cu") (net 5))
 (segment (start 56.47625 -3.546212) (end 54.692462 -5.33) (width 1) (layer "B.Cu") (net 5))
 (segment (start 2.6 55.2125) (end -9.8925 42.72) (width 1) (layer "B.Cu") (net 5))
 (segment (start 30.31 37.72) (end 25.41 37.72) (width 1) (layer "B.Cu") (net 5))
 (segment (start 9.71 42.72) (end 14.03 47.04) (width 1) (layer "B.Cu") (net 5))
 (segment (start -9.8925 42.72) (end -25.91 42.72) (width 1) (layer "B.Cu") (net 5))
 (segment (start 60.23 16.8275) (end 56.47625 13.07375) (width 1) (layer "B.Cu") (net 5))
 (segment (start -20.192 -22.70647) (end -20.192 -16.941) (width 1) (layer "B.Cu") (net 5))
 (segment (start 9.71 42.72) (end 10.81 42.72) (width 1) (layer "B.Cu") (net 5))
 (segment (start 25.33 47.04) (end 25.33 37.8) (width 1) (layer "B.Cu") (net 5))
 (segment (start -25.91 42.72) (end -25.91 -0.2725) (width 1) (layer "B.Cu") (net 5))
 (segment (start 30.31 37.72) (end 41.87 37.72) (width 1) (layer "B.Cu") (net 5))
 (segment (start 56.47625 13.07375) (end 54.4225 11.02) (width 1) (layer "B.Cu") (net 5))
 (segment (start 14.03 47.04) (end 25.33 47.04) (width 1) (layer "B.Cu") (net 5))
 (segment (start -11.36 -28.8) (end -14.09847 -28.8) (width 1) (layer "B.Cu") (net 5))
 (segment (start 46.1925 19.25) (end 43.94 19.25) (width 1) (layer "B.Cu") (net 5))
 (segment (start -20.192 -16.941) (end -21.643 -15.49) (width 1) (layer "B.Cu") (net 5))
 (segment (start -18.83 -12.677) (end -18.83 -7.3525) (width 1) (layer "B.Cu") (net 5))
 (segment (start -14.09847 -28.8) (end -20.192 -22.70647) (width 1) (layer "B.Cu") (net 5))
 (segment (start 52.13625 13.30625) (end 46.1925 19.25) (width 1) (layer "B.Cu") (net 5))
 (segment (start 60.23 19.36) (end 60.23 16.8275) (width 1) (layer "B.Cu") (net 5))
 (segment (start -11.36 -28.8) (end -11.36 -41.257) (width 1) (layer "B.Cu") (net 5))
 (segment (start 56.47625 13.07375) (end 56.47625 -3.546212) (width 1) (layer "B.Cu") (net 5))
 (segment (start -10.283 -27.337) (end -9.897 -27.337) (width 1) (layer "B.Cu") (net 12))
 (segment (start 8.09 35.18) (end -16.89 10.2) (width 1) (layer "B.Cu") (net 12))
 (segment (start 20.15 35.18) (end 8.09 35.18) (width 1) (layer "B.Cu") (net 12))
 (segment (start -14.93 -26.27) (end -14.92 -26.26) (width 1) (layer "B.Cu") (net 12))
 (segment (start 38.42 -30.52) (end 59.7 -9.24) (width 1) (layer "B.Cu") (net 12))
 (segment (start -14.92 -26.26) (end -11.36 -26.26) (width 1) (layer "B.Cu") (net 12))
 (segment (start -9.897 -27.337) (end -9.897 -27.723) (width 1) (layer "B.Cu") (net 12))
 (segment (start -7.1 -30.52) (end 38.42 -30.52) (width 1) (layer "B.Cu") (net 12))
 (segment (start 57.06 -6.6) (end 53.95 -6.6) (width 1) (layer "B.Cu") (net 12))
 (segment (start -14.93 8.24) (end -14.93 -26.27) (width 1) (layer "B.Cu") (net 12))
 (segment (start -9.897 -27.723) (end -7.1 -30.52) (width 1) (layer "B.Cu") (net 12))
 (segment (start 59.7 -9.24) (end 57.06 -6.6) (width 1) (layer "B.Cu") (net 12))
 (segment (start -11.36 -26.26) (end -10.283 -27.337) (width 1) (layer "B.Cu") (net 12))
 (segment (start -16.89 10.2) (end -14.93 8.24) (width 1) (layer "B.Cu") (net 12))
 (segment (start -26.14 -36.47) (end -26.04 -36.47) (width 1) (layer "B.Cu") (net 6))
 (segment (start 44.03 26.67) (end 38.82 26.67) (width 1) (layer "B.Cu") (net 6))
 (segment (start -23.66 -10.41) (end -37.93 -24.68) (width 1) (layer "B.Cu") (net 6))
 (segment (start 54.4225 16.02) (end 54.4225 16.2775) (width 1) (layer "B.Cu") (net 6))
 (segment (start 52.68 -7.87) (end 53.95 -7.87) (width 1) (layer "B.Cu") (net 6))
 (segment (start 30.31 35.18) (end 38.82 26.67) (width 1) (layer "B.Cu") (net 6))
 (segment (start 11.44 26.67) (end 9.71 24.94) (width 1) (layer "B.Cu") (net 6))
 (segment (start -5.93 9.3) (end -11.36 9.3) (width 1) (layer "B.Cu") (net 6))
 (segment (start 9.71 24.94) (end -5.93 9.3) (width 1) (layer "B.Cu") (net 6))
 (segment (start -23.66 -10.41) (end -23.66 -9.87) (width 1) (layer "B.Cu") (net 6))
 (segment (start 43.94 21.79) (end 43.94 23.68) (width 1) (layer "B.Cu") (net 6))
 (segment (start 9.71 24.94) (end 9.71 18.5) (width 1) (layer "B.Cu") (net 6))
 (segment (start -23.66 -9.87) (end -29.7525 -3.7775) (width 1) (layer "B.Cu") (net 6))
 (segment (start 54.4225 16.2775) (end 45.48 25.22) (width 1) (layer "B.Cu") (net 6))
 (segment (start 40.24 -7.87) (end 52.68 -7.87) (width 1) (layer "B.Cu") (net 6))
 (segment (start 45.48 25.22) (end 44.03 26.67) (width 1) (layer "B.Cu") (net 6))
 (segment (start -37.93 -24.68) (end -26.14 -36.47) (width 1) (layer "B.Cu") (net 6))
 (segment (start -26.04 -36.47) (end -20.18 -42.33) (width 1) (layer "B.Cu") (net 6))
 (segment (start -23.66 -10.41) (end -21.643 -10.41) (width 1) (layer "B.Cu") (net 6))
 (segment (start 9.71 18.5) (end 13.87 18.5) (width 1) (layer "B.Cu") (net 6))
 (segment (start 38.82 26.67) (end 11.44 26.67) (width 1) (layer "B.Cu") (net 6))
 (segment (start -29.7525 -3.7775) (end -29.7525 1.03) (width 1) (layer "B.Cu") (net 6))
 (segment (start 43.94 23.68) (end 45.48 25.22) (width 1) (layer "B.Cu") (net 6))
 (segment (start -20.18 -42.33) (end -14.973 -42.33) (width 1) (layer "B.Cu") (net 6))
 (segment (start 13.87 18.5) (end 40.24 -7.87) (width 1) (layer "B.Cu") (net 6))
 (segment (start 21.304 31.486) (end 21.304 29.621997) (width 0.406) (layer "F.Cu") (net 13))
 (segment (start -4.097997 4.22) (end -11.36 4.22) (width 0.406) (layer "F.Cu") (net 13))
 (segment (start 21.304 29.621997) (end -4.097997 4.22) (width 0.406) (layer "F.Cu") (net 13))
 (segment (start 20.15 32.64) (end 21.304 31.486) (width 0.406) (layer "F.Cu") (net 13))
 (segment (start 11.98 30.1) (end -11.36 6.76) (width 0.406) (layer "F.Cu") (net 14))
 (segment (start 20.15 30.1) (end 11.98 30.1) (width 0.406) (layer "F.Cu") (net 14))
 (segment (start 8.717 -26.26) (end -14.973 -49.95) (width 0.406) (layer "F.Cu") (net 26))
 (segment (start 11.5 -26.26) (end 8.717 -26.26) (width 0.406) (layer "F.Cu") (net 26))
 (segment (start 8.717 -23.72) (end -14.973 -47.41) (width 0.406) (layer "F.Cu") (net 27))
 (segment (start 11.5 -23.72) (end 8.717 -23.72) (width 0.406) (layer "F.Cu") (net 27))
 (segment (start 38.05 11.84) (end 52.68 -2.79) (width 0.406) (layer "F.Cu") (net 39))
 (segment (start 11.5 11.84) (end 38.05 11.84) (width 0.406) (layer "F.Cu") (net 39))
 (segment (start 11.5 6.76) (end 34.44 6.76) (width 0.406) (layer "F.Cu") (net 37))
 (segment (start 46.53 -5.33) (end 52.68 -5.33) (width 0.406) (layer "F.Cu") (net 37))
 (segment (start 34.44 6.76) (end 46.53 -5.33) (width 0.406) (layer "F.Cu") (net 37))
 (segment (start 33.07 4.22) (end 44.55 -7.26) (width 0.406) (layer "F.Cu") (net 36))
 (segment (start 45.21 -6.6) (end 52.68 -6.6) (width 0.406) (layer "F.Cu") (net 36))
 (segment (start 11.5 4.22) (end 33.07 4.22) (width 0.406) (layer "F.Cu") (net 36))
 (segment (start 44.55 -7.26) (end 45.21 -6.6) (width 0.406) (layer "F.Cu") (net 36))
 (segment (start 51.13 -4.06) (end 52.68 -4.06) (width 0.406) (layer "F.Cu") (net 38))
 (segment (start 11.5 9.3) (end 37.77 9.3) (width 0.406) (layer "F.Cu") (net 38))
 (segment (start 37.77 9.3) (end 51.13 -4.06) (width 0.406) (layer "F.Cu") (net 38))
 (segment (start -44.9925 16.27) (end -36.0365 7.314) (width 0.406) (layer "F.Cu") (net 24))
 (segment (start -36.0365 7.314) (end -19.534 7.314) (width 0.406) (layer "F.Cu") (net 24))
 (segment (start -19.534 7.314) (end -11.36 -0.86) (width 0.406) (layer "F.Cu") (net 24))
 (segment (start -29.7525 16.27) (end -25.95 16.27) (width 0.406) (layer "F.Cu") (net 25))
 (segment (start -25.95 16.27) (end -11.36 1.68) (width 0.406) (layer "F.Cu") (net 25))
 (segment (start -30.93 34.14) (end -30.93 24.94) (width 1) (layer "B.Cu") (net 7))
 (segment (start 7.6 55.2125) (end 4.7225 58.09) (width 1) (layer "B.Cu") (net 7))
 (segment (start -37.7 40.91) (end -30.93 34.14) (width 1) (layer "B.Cu") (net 7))
 (segment (start 4.7225 58.09) (end -20.52 58.09) (width 1) (layer "B.Cu") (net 7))
 (segment (start -20.52 58.09) (end -37.7 40.91) (width 1) (layer "B.Cu") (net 7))
 (segment (start -1.0675 48.88) (end 24.02 48.88) (width 0.406) (layer "F.Cu") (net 1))
 (segment (start -7.4 55.2125) (end -1.0675 48.88) (width 0.406) (layer "F.Cu") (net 1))
 (segment (start 24.02 48.88) (end 24.02 29.01) (width 0.406) (layer "F.Cu") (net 1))
 (segment (start 24.02 29.01) (end 43.94 9.09) (width 0.406) (layer "F.Cu") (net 1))
 (segment (start -2.4 55.2125) (end 1.4725 51.34) (width 0.406) (layer "F.Cu") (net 2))
 (segment (start 26.42 29.15) (end 43.94 11.63) (width 0.406) (layer "F.Cu") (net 2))
 (segment (start 26.42 51.34) (end 26.42 29.15) (width 0.406) (layer "F.Cu") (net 2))
 (segment (start 1.4725 51.34) (end 26.42 51.34) (width 0.406) (layer "F.Cu") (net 2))
 (segment (start 43.7 16.71) (end 43.94 16.71) (width 0.406) (layer "F.Cu") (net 4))
 (segment (start 30.31 30.1) (end 43.7 16.71) (width 0.406) (layer "F.Cu") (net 4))
 (segment (start 28.78 29.33) (end 43.94 14.17) (width 0.406) (layer "F.Cu") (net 3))
 (segment (start 30.31 32.64) (end 28.58 30.91) (width 0.406) (layer "F.Cu") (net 3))
 (segment (start 28.58 29.88) (end 28.78 29.68) (width 0.406) (layer "F.Cu") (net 3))
 (segment (start 28.78 29.68) (end 28.78 29.33) (width 0.406) (layer "F.Cu") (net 3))
 (segment (start 28.58 30.91) (end 28.58 29.88) (width 0.406) (layer "F.Cu") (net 3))
 (segment (start 11.5 -21.18) (end 46.87 -21.18) (width 0.406) (layer "F.Cu") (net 22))
 (segment (start 54.59 -2.15) (end 53.95 -2.79) (width 0.406) (layer "F.Cu") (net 22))
 (segment (start 61.85 -6.2) (end 61.85 -2.15) (width 0.406) (layer "F.Cu") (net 22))
 (segment (start 61.85 -2.15) (end 54.59 -2.15) (width 0.406) (layer "F.Cu") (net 22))
 (segment (start 46.87 -21.18) (end 61.85 -6.2) (width 0.406) (layer "F.Cu") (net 22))
 (segment (start 58.5 -4.06) (end 53.95 -4.06) (width 0.406) (layer "F.Cu") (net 23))
 (segment (start 45.8 -18.64) (end 59.44 -5) (width 0.406) (layer "F.Cu") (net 23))
 (segment (start 11.5 -18.64) (end 45.8 -18.64) (width 0.406) (layer "F.Cu") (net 23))
 (segment (start 59.44 -5) (end 58.5 -4.06) (width 0.406) (layer "F.Cu") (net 23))
 (segment (start -21.643 -20.57) (end -13.467 -12.394) (width 0.406) (layer "F.Cu") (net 30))
 (segment (start 10.126 -12.394) (end 11.5 -11.02) (width 0.406) (layer "F.Cu") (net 30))
 (segment (start -13.467 -12.394) (end 10.126 -12.394) (width 0.406) (layer "F.Cu") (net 30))
 (segment (start -21.643 -18.03) (end -13.467 -9.854) (width 0.406) (layer "F.Cu") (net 31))
 (segment (start -13.467 -9.854) (end 10.126 -9.854) (width 0.406) (layer "F.Cu") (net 31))
 (segment (start 10.126 -9.854) (end 11.5 -8.48) (width 0.406) (layer "F.Cu") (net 31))
 (segment (start -13.467 -14.934) (end 10.126 -14.934) (width 0.406) (layer "F.Cu") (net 29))
 (segment (start 10.126 -14.934) (end 11.5 -13.56) (width 0.406) (layer "F.Cu") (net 29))
 (segment (start -21.643 -23.11) (end -13.467 -14.934) (width 0.406) (layer "F.Cu") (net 29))
 (segment (start -13.433 -17.44) (end 10.16 -17.44) (width 0.406) (layer "F.Cu") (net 28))
 (segment (start -21.643 -25.65) (end -13.433 -17.44) (width 0.406) (layer "F.Cu") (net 28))
 (segment (start 10.16 -17.44) (end 11.5 -16.1) (width 0.406) (layer "F.Cu") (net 28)))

